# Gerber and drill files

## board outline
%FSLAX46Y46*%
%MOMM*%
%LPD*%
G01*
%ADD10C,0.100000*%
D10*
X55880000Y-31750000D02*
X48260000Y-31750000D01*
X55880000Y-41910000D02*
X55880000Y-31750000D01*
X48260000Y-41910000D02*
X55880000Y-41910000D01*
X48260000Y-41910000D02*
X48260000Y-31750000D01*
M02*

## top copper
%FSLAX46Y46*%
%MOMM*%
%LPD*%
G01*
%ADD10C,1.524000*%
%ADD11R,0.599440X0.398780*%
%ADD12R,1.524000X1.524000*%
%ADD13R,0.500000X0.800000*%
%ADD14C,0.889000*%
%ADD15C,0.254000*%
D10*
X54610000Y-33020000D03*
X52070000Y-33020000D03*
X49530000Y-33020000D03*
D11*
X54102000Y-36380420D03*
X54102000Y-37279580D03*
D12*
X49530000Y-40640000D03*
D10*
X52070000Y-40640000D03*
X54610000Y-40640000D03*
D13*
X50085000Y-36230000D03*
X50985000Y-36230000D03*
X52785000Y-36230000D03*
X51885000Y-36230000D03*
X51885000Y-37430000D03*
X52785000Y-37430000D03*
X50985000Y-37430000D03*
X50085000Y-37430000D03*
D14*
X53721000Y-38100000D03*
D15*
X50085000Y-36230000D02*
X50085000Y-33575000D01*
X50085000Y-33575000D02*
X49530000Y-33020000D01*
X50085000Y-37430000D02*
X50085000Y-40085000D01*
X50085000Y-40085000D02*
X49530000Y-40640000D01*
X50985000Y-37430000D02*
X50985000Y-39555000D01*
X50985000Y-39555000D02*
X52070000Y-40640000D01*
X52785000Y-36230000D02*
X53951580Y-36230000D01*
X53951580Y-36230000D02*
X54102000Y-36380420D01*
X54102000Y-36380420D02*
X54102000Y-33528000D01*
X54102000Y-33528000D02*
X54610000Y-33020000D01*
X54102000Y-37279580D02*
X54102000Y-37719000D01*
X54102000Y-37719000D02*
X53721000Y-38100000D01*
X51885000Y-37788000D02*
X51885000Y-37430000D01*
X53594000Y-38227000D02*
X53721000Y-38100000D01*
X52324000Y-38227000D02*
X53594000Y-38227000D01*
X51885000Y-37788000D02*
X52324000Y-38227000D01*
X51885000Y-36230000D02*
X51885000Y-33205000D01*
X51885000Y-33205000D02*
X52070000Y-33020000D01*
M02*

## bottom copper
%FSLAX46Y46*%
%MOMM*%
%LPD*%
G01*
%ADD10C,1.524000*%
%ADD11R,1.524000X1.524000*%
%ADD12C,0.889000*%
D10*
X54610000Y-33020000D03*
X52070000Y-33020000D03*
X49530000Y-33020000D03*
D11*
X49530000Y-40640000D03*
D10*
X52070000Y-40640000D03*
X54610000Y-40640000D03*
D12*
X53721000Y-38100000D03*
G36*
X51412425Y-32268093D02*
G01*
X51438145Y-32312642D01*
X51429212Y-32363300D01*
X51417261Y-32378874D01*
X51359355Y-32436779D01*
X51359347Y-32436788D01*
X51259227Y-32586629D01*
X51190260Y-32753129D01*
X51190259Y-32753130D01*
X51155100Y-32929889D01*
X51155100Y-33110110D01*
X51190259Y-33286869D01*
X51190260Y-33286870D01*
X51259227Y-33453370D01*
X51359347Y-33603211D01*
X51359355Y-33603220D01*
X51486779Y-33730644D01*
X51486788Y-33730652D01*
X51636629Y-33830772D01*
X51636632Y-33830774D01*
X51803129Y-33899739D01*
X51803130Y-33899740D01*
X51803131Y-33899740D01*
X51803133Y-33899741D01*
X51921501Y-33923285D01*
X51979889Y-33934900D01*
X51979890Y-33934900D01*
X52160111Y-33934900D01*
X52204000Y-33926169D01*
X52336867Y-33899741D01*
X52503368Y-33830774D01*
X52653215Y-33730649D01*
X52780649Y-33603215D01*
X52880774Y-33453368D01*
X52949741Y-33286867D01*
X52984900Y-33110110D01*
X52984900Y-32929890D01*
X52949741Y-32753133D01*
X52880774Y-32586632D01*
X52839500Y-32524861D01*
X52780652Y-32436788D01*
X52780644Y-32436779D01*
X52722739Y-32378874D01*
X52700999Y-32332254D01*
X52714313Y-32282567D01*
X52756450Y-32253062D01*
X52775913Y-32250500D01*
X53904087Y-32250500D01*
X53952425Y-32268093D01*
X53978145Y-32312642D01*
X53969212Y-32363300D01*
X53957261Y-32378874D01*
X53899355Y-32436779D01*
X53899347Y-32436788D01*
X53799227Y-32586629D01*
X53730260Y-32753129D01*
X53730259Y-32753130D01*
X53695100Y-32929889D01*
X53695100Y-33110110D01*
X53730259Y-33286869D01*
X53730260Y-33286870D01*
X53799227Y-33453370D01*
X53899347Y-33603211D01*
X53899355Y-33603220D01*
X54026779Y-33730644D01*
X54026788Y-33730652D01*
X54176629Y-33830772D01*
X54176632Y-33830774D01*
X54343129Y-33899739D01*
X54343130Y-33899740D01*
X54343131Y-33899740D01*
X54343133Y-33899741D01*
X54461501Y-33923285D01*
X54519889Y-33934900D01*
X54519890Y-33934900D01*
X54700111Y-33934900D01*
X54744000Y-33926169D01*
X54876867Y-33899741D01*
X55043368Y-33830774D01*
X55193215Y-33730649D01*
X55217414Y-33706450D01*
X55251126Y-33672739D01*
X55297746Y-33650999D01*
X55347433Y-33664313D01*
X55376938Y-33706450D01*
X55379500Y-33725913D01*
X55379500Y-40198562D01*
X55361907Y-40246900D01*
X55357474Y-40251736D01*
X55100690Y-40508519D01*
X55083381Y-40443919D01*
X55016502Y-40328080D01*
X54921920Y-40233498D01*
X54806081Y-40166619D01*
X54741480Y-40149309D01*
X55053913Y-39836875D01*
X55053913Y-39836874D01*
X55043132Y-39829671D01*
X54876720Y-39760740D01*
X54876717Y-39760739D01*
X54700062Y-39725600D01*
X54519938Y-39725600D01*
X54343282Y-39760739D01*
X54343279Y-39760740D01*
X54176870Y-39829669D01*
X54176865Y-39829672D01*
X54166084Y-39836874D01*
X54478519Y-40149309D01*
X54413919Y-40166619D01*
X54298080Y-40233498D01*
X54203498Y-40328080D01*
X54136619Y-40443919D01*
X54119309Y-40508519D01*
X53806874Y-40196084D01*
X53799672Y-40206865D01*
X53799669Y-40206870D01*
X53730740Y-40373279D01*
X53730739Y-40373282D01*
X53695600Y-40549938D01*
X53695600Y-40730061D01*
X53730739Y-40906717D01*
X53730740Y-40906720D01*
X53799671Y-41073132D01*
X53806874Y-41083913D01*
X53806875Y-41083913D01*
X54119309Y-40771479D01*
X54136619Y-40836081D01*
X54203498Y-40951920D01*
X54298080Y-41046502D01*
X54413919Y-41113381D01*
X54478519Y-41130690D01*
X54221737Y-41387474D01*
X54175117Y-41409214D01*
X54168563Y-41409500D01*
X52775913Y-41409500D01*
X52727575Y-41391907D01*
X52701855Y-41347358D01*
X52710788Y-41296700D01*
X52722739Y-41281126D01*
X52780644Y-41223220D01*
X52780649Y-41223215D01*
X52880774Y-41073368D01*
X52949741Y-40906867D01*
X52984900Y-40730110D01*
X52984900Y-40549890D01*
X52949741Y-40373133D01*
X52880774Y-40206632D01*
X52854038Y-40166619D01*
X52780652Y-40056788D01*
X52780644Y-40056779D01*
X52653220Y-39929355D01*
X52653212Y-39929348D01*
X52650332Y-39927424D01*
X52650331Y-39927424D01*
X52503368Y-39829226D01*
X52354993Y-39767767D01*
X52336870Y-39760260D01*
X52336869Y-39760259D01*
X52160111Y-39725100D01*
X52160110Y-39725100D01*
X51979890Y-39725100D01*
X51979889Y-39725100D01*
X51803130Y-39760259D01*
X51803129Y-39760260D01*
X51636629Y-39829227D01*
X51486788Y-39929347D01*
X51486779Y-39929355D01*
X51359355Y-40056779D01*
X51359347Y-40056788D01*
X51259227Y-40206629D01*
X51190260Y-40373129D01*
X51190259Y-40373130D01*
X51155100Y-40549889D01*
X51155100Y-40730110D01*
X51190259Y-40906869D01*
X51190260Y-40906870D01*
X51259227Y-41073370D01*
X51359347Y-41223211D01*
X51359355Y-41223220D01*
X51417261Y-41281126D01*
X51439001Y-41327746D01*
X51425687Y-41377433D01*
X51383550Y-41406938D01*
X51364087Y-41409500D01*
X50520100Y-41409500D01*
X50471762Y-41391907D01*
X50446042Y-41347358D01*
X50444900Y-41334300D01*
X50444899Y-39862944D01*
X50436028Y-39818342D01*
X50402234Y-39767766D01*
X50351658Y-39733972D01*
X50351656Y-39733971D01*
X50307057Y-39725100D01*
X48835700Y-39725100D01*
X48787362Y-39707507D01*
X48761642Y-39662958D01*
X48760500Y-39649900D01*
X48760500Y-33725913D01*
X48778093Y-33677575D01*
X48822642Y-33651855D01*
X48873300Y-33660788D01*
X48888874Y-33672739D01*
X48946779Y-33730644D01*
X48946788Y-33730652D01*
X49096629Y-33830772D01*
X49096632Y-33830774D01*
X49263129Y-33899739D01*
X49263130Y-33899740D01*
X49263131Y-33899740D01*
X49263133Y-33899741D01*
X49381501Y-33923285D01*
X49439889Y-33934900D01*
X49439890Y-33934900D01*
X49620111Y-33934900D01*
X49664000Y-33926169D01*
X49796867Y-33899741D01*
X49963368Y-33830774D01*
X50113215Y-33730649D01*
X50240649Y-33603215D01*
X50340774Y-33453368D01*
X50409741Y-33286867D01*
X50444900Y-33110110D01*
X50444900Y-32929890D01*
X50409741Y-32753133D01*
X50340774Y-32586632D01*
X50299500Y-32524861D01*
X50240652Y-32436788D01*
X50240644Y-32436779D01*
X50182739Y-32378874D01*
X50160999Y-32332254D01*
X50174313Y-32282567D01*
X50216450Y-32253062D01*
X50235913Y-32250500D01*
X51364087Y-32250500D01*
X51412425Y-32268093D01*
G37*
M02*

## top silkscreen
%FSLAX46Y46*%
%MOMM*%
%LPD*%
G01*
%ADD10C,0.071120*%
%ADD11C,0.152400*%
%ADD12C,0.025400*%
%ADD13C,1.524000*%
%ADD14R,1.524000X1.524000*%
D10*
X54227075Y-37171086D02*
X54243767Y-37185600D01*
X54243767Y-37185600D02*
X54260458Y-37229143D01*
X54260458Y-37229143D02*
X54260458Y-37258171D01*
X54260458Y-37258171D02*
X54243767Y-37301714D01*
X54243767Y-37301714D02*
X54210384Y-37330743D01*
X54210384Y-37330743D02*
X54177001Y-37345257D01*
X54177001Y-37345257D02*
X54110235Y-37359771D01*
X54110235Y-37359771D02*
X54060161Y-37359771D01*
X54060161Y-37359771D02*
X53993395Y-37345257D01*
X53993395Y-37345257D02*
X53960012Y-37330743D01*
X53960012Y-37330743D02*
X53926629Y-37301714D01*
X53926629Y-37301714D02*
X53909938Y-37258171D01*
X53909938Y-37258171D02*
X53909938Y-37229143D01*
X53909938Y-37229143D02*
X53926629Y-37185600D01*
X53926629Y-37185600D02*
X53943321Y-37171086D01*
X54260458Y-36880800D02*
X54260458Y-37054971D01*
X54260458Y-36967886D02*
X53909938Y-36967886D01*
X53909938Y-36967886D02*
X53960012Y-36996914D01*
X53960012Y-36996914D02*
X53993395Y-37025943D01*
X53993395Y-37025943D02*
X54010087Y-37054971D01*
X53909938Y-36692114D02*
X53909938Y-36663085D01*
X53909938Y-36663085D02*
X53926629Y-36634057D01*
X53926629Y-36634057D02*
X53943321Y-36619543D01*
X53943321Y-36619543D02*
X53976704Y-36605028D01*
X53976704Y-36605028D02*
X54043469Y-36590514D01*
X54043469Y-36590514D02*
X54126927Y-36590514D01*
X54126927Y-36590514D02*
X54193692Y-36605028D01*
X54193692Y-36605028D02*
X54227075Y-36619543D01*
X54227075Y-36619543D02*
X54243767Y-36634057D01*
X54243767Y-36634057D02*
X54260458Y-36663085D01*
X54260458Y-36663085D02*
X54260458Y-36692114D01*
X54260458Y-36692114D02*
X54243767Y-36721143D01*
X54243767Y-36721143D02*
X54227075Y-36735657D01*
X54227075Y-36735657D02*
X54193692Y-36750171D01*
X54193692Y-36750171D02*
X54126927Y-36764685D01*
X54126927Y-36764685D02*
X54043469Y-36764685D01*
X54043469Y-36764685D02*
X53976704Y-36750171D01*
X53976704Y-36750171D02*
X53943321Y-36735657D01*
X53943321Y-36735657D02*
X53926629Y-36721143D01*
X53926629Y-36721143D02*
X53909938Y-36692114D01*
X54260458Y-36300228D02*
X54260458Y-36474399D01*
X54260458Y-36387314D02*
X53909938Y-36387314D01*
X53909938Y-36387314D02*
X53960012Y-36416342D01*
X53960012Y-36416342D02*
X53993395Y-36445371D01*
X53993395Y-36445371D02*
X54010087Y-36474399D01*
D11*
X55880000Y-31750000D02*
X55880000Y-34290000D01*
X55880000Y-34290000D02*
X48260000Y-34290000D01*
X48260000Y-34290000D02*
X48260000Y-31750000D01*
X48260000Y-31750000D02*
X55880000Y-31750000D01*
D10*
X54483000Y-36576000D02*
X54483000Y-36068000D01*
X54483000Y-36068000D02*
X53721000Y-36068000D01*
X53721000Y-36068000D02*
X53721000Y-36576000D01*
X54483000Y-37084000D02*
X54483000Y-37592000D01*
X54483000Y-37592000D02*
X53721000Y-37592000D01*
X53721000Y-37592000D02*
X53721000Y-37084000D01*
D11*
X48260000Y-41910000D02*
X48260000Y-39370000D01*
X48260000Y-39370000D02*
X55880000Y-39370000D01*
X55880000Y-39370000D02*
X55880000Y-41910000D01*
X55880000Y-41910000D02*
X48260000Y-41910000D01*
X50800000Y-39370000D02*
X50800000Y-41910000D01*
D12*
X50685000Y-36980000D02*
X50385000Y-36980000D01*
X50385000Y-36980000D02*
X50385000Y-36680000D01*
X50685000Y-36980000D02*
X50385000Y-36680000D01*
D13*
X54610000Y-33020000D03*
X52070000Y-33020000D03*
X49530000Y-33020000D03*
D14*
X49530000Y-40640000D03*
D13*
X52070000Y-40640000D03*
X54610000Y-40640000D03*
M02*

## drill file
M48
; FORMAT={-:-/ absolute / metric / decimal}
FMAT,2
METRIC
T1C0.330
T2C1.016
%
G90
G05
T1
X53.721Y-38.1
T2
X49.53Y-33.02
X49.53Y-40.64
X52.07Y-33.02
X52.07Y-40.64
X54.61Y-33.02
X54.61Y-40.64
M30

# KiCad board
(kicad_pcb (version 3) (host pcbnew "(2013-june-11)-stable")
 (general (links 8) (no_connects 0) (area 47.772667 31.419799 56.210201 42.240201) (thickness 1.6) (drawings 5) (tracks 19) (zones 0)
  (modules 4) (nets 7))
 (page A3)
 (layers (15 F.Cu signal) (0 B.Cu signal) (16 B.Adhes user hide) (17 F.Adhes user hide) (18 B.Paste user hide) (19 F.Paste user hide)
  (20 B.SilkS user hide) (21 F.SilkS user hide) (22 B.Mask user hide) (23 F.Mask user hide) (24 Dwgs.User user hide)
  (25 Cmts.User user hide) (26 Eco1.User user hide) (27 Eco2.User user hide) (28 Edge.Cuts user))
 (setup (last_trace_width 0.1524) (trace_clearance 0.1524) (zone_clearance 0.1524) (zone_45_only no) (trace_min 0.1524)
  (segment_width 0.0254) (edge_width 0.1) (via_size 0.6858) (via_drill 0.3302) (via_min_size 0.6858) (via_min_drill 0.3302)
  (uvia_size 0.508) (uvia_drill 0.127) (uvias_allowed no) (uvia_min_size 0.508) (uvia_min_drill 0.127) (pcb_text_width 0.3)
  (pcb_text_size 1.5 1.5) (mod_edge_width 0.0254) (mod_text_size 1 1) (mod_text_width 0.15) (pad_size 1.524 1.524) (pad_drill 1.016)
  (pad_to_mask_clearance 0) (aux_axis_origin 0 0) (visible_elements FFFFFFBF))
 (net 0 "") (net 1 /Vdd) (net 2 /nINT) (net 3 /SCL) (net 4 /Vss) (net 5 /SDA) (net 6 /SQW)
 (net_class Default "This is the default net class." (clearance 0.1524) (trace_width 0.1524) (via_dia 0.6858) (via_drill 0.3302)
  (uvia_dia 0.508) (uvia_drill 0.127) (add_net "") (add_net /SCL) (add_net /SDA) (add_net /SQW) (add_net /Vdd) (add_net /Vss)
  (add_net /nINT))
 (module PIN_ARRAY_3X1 (layer F.Cu) (at 52.07 33.02 180)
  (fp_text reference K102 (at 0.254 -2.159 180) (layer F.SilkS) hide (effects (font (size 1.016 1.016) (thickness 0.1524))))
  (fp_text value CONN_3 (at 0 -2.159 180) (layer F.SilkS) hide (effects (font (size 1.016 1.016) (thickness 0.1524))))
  (fp_line (start -3.81 1.27) (end -3.81 -1.27) (layer F.SilkS) (width 0.1524))
  (fp_line (start -3.81 -1.27) (end 3.81 -1.27) (layer F.SilkS) (width 0.1524))
  (fp_line (start 3.81 -1.27) (end 3.81 1.27) (layer F.SilkS) (width 0.1524))
  (fp_line (start 3.81 1.27) (end -3.81 1.27) (layer F.SilkS) (width 0.1524))
  (pad 1 thru_hole circle (at -2.54 0 180) (size 1.524 1.524) (drill 1.016) (layers *.Cu *.Mask F.SilkS) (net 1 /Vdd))
  (pad 2 thru_hole circle (at 0 0 180) (size 1.524 1.524) (drill 1.016) (layers *.Cu *.Mask F.SilkS) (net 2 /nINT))
  (pad 3 thru_hole circle (at 2.54 0 180) (size 1.524 1.524) (drill 1.016) (layers *.Cu *.Mask F.SilkS) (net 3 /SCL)))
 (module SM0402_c (layer F.Cu) (at 54.102 36.83 270)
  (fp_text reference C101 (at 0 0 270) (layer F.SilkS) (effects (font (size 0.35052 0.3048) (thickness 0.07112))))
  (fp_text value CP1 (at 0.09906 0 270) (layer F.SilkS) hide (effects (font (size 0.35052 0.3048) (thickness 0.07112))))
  (fp_line (start -0.254 -0.381) (end -0.762 -0.381) (layer F.SilkS) (width 0.07112))
  (fp_line (start -0.762 -0.381) (end -0.762 0.381) (layer F.SilkS) (width 0.07112))
  (fp_line (start -0.762 0.381) (end -0.254 0.381) (layer F.SilkS) (width 0.07112))
  (fp_line (start 0.254 -0.381) (end 0.762 -0.381) (layer F.SilkS) (width 0.07112))
  (fp_line (start 0.762 -0.381) (end 0.762 0.381) (layer F.SilkS) (width 0.07112))
  (fp_line (start 0.762 0.381) (end 0.254 0.381) (layer F.SilkS) (width 0.07112))
  (pad 1 smd rect (at -0.44958 0 270) (size 0.39878 0.59944) (layers F.Cu F.Paste F.Mask) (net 1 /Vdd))
  (pad 2 smd rect (at 0.44958 0 270) (size 0.39878 0.59944) (layers F.Cu F.Paste F.Mask) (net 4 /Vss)))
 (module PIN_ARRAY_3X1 (layer F.Cu) (at 52.07 40.64)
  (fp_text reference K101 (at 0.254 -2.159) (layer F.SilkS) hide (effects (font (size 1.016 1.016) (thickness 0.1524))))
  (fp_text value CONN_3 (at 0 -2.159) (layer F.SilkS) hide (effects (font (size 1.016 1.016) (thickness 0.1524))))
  (fp_line (start -3.81 1.27) (end -3.81 -1.27) (layer F.SilkS) (width 0.1524))
  (fp_line (start -3.81 -1.27) (end 3.81 -1.27) (layer F.SilkS) (width 0.1524))
  (fp_line (start 3.81 -1.27) (end 3.81 1.27) (layer F.SilkS) (width 0.1524))
  (fp_line (start 3.81 1.27) (end -3.81 1.27) (layer F.SilkS) (width 0.1524))
  (fp_line (start -1.27 -1.27) (end -1.27 1.27) (layer F.SilkS) (width 0.1524))
  (pad 1 thru_hole rect (at -2.54 0) (size 1.524 1.524) (drill 1.016) (layers *.Cu *.Mask F.SilkS) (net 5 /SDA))
  (pad 2 thru_hole circle (at 0 0) (size 1.524 1.524) (drill 1.016) (layers *.Cu *.Mask F.SilkS) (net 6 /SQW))
  (pad 3 thru_hole circle (at 2.54 0) (size 1.524 1.524) (drill 1.016) (layers *.Cu *.Mask F.SilkS) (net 4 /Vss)))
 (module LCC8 (layer F.Cu) (at 51.435 36.83)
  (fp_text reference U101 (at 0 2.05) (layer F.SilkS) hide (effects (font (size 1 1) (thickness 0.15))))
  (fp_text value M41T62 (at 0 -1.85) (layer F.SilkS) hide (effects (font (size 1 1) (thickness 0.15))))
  (fp_line (start -0.75 0.15) (end -1.05 0.15) (layer F.SilkS) (width 0.0254))
  (fp_line (start -1.05 0.15) (end -1.05 -0.15) (layer F.SilkS) (width 0.0254))
  (fp_line (start -0.75 0.15) (end -1.05 -0.15) (layer F.SilkS) (width 0.0254))
  (pad 8 smd rect (at -1.35 -0.6) (size 0.5 0.8) (layers F.Cu F.Paste F.Mask) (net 3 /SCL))
  (pad 7 smd rect (at -0.45 -0.6) (size 0.5 0.8) (layers F.Cu F.Paste F.Mask))
  (pad 5 smd rect (at 1.35 -0.6) (size 0.5 0.8) (layers F.Cu F.Paste F.Mask) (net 1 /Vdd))
  (pad 6 smd rect (at 0.45 -0.6) (size 0.5 0.8) (layers F.Cu F.Paste F.Mask) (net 2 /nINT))
  (pad 3 smd rect (at 0.45 0.6) (size 0.5 0.8) (layers F.Cu F.Paste F.Mask) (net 4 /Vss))
  (pad 4 smd rect (at 1.35 0.6) (size 0.5 0.8) (layers F.Cu F.Paste F.Mask))
  (pad 2 smd rect (at -0.45 0.6) (size 0.5 0.8) (layers F.Cu F.Paste F.Mask) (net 6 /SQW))
  (pad 1 smd rect (at -1.35 0.6) (size 0.5 0.8) (layers F.Cu F.Paste F.Mask) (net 5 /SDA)))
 (gr_line (start 55.88 31.75) (end 48.26 31.75) (angle 90) (layer Edge.Cuts) (width 0.1))
 (gr_line (start 55.88 41.91) (end 55.88 31.75) (angle 90) (layer Edge.Cuts) (width 0.1))
 (gr_line (start 48.26 41.91) (end 55.88 41.91) (angle 90) (layer Edge.Cuts) (width 0.1))
 (gr_line (start 48.26 41.91) (end 48.26 31.75) (angle 90) (layer Edge.Cuts) (width 0.1))
 (segment (start 50.085 36.23) (end 50.085 33.575) (width 0.254) (layer F.Cu) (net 3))
 (segment (start 50.085 33.575) (end 49.53 33.02) (width 0.254) (layer F.Cu) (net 3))
 (segment (start 50.085 37.43) (end 50.085 40.085) (width 0.254) (layer F.Cu) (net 5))
 (segment (start 50.085 40.085) (end 49.53 40.64) (width 0.254) (layer F.Cu) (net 5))
 (segment (start 50.985 37.43) (end 50.985 39.555) (width 0.254) (layer F.Cu) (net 6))
 (segment (start 50.985 39.555) (end 52.07 40.64) (width 0.254) (layer F.Cu) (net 6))
 (segment (start 52.785 36.23) (end 53.95158 36.23) (width 0.254) (layer F.Cu) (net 1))
 (segment (start 53.95158 36.23) (end 54.102 36.38042) (width 0.254) (layer F.Cu) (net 1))
 (segment (start 54.102 36.38042) (end 54.102 33.528) (width 0.254) (layer F.Cu) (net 1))
 (segment (start 54.102 33.528) (end 54.61 33.02) (width 0.254) (layer F.Cu) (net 1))
 (segment (start 54.102 37.27958) (end 54.102 37.719) (width 0.254) (layer F.Cu) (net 4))
 (segment (start 54.102 37.719) (end 53.721 38.1) (width 0.254) (layer F.Cu) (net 4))
 (segment (start 51.885 37.788) (end 51.885 37.43) (width 0.254) (layer F.Cu) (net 4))
 (via (at 53.721 38.1) (size 0.889) (layers F.Cu B.Cu) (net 4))
 (segment (start 53.594 38.227) (end 53.721 38.1) (width 0.254) (layer F.Cu) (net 4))
 (segment (start 52.324 38.227) (end 53.594 38.227) (width 0.254) (layer F.Cu) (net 4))
 (segment (start 51.885 37.788) (end 52.324 38.227) (width 0.254) (layer F.Cu) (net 4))
 (segment (start 51.885 36.23) (end 51.885 33.205) (width 0.254) (layer F.Cu) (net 2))
 (segment (start 51.885 33.205) (end 52.07 33.02) (width 0.254) (layer F.Cu) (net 2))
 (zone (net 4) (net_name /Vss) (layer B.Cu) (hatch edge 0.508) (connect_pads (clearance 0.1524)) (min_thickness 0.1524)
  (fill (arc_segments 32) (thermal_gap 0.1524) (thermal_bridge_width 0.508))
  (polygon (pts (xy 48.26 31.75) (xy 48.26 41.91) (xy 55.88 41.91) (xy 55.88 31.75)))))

